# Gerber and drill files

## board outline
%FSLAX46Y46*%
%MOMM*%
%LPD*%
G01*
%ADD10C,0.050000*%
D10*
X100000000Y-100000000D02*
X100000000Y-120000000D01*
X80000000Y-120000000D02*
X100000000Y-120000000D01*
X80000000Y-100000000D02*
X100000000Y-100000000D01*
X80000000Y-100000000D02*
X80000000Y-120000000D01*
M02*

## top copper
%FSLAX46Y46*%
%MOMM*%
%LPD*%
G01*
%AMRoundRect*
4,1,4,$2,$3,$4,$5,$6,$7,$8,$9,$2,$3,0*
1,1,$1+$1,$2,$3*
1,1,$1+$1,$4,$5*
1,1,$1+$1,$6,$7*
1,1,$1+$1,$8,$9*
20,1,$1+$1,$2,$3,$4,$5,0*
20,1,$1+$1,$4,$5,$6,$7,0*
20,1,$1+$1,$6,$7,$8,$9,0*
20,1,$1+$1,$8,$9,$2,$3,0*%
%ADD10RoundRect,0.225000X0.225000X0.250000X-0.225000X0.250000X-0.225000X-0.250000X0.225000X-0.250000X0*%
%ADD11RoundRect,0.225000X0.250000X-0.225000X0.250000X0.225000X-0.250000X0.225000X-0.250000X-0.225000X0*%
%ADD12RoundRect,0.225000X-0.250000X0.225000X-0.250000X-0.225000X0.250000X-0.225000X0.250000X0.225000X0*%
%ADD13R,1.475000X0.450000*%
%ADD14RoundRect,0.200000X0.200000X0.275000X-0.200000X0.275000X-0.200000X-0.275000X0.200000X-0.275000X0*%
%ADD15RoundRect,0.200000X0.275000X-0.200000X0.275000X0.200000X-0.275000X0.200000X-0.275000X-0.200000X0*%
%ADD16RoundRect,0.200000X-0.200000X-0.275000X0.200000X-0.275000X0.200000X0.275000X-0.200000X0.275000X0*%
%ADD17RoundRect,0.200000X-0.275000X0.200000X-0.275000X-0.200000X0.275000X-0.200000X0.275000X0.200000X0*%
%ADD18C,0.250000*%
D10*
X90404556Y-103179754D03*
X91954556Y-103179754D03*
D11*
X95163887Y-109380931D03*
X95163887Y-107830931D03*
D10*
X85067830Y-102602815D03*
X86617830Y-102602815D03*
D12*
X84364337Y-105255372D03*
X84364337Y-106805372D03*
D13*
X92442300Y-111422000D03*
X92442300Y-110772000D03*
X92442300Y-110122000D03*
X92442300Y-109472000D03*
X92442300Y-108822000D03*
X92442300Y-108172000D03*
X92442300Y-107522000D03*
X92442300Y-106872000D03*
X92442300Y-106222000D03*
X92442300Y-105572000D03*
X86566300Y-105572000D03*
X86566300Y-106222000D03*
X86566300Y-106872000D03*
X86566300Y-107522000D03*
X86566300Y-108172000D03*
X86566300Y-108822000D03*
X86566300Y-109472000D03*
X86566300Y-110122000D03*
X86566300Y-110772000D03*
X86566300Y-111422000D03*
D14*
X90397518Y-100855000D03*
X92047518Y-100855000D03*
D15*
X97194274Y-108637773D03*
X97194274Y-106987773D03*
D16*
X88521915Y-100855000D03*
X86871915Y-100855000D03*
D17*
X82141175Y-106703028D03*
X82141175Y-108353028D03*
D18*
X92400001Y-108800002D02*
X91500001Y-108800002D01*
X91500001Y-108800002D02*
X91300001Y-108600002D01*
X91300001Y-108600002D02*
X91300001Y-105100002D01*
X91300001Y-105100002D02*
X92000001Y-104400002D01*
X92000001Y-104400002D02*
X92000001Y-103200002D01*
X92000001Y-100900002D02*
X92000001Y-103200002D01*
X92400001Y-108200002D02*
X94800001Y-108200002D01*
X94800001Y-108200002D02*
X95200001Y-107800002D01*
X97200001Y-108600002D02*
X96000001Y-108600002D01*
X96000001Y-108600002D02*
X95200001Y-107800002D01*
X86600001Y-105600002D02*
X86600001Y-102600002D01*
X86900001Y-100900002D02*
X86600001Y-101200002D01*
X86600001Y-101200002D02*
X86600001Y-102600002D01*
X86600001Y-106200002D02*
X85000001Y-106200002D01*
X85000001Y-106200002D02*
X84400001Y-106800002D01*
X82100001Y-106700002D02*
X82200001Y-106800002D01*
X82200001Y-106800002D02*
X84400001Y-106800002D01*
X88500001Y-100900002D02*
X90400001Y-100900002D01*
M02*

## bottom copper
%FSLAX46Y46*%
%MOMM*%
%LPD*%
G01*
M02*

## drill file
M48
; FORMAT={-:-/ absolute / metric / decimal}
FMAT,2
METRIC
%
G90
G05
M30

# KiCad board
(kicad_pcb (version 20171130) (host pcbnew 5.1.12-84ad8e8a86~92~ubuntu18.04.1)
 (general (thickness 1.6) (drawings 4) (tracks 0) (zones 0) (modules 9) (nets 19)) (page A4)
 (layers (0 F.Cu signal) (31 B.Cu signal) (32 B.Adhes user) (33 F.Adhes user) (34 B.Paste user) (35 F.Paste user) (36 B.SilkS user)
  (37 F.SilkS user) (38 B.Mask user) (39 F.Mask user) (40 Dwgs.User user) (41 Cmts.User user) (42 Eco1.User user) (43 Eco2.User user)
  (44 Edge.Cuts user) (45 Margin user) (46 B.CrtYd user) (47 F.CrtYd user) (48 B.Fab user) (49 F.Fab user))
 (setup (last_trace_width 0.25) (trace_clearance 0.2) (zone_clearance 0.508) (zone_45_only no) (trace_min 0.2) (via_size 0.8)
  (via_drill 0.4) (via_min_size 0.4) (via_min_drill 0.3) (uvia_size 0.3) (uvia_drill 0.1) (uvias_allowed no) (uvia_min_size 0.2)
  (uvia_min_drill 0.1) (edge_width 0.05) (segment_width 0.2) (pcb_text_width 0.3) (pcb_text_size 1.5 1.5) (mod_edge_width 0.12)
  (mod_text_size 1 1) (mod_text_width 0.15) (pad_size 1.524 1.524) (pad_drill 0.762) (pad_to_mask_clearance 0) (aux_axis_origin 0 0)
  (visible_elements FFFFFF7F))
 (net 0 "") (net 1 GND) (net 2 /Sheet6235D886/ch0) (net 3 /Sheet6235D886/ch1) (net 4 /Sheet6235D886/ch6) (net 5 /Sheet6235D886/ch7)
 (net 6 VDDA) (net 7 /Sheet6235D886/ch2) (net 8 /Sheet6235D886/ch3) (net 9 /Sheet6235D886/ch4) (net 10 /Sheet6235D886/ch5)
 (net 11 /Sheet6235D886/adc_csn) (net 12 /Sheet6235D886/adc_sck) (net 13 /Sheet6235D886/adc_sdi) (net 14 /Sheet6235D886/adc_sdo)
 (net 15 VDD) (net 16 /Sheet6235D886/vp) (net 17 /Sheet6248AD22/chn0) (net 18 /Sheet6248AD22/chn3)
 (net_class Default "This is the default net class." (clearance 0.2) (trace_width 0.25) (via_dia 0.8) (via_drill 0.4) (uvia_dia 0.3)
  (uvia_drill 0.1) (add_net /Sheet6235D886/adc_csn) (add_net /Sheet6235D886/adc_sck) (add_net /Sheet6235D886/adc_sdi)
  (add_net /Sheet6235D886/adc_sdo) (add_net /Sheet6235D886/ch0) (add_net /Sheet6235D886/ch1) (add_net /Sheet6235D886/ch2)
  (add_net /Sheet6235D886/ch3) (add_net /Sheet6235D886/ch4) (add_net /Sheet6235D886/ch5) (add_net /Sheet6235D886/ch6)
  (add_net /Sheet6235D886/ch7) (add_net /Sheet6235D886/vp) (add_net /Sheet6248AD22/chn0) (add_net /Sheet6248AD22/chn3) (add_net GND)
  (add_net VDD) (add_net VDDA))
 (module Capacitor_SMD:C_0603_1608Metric (layer F.Cu) (at 91.179556 103.179754 180.000000)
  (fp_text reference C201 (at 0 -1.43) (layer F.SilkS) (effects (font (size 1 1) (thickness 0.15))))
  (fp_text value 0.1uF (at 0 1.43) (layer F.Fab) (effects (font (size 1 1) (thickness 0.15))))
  (pad 2 smd roundrect (at 0.775 0 180.000000) (size 0.9 0.95) (layers F.Cu F.Mask F.Paste) (roundrect_rratio 0.25) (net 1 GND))
  (pad 1 smd roundrect (at -0.775 0 180.000000) (size 0.9 0.95) (layers F.Cu F.Mask F.Paste) (roundrect_rratio 0.25)
   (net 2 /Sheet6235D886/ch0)))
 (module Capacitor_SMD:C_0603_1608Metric (layer F.Cu) (at 95.163887 108.605931 90.000000)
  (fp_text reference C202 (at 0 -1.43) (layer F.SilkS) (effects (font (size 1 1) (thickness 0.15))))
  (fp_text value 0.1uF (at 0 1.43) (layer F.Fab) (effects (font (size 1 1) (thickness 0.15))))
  (pad 1 smd roundrect (at -0.775 0 90.000000) (size 0.9 0.95) (layers F.Cu F.Mask F.Paste) (roundrect_rratio 0.25) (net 1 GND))
  (pad 2 smd roundrect (at 0.775 0 90.000000) (size 0.9 0.95) (layers F.Cu F.Mask F.Paste) (roundrect_rratio 0.25)
   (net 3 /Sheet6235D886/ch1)))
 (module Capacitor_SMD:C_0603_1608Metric (layer F.Cu) (at 85.842830 102.602815 180.000000)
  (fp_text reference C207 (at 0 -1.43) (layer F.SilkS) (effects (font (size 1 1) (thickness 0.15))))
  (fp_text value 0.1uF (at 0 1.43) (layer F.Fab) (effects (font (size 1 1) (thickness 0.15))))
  (pad 2 smd roundrect (at 0.775 0 180.000000) (size 0.9 0.95) (layers F.Cu F.Mask F.Paste) (roundrect_rratio 0.25) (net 1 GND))
  (pad 1 smd roundrect (at -0.775 0 180.000000) (size 0.9 0.95) (layers F.Cu F.Mask F.Paste) (roundrect_rratio 0.25)
   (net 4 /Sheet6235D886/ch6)))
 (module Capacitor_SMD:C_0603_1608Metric (layer F.Cu) (at 84.364337 106.030372 270.000000)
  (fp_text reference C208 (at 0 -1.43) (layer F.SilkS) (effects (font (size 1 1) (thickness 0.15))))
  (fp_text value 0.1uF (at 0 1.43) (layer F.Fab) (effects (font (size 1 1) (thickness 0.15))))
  (pad 1 smd roundrect (at -0.775 0 270.000000) (size 0.9 0.95) (layers F.Cu F.Mask F.Paste) (roundrect_rratio 0.25) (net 1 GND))
  (pad 2 smd roundrect (at 0.775 0 270.000000) (size 0.9 0.95) (layers F.Cu F.Mask F.Paste) (roundrect_rratio 0.25)
   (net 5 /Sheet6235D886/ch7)))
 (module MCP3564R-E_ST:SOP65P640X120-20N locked (layer F.Cu) (at 89.504300 108.497000 180.000000)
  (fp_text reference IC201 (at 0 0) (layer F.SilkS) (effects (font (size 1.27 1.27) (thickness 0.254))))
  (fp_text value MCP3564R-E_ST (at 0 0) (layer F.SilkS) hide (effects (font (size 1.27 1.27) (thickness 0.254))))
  (pad 1 smd rect (at -2.938 -2.925 270.000000) (size 0.45 1.475) (layers F.Cu F.Mask F.Paste) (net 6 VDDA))
  (pad 2 smd rect (at -2.938 -2.275 270.000000) (size 0.45 1.475) (layers F.Cu F.Mask F.Paste) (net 1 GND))
  (pad 3 smd rect (at -2.938 -1.625 270.000000) (size 0.45 1.475) (layers F.Cu F.Mask F.Paste) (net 1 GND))
  (pad 4 smd rect (at -2.938 -0.975 270.000000) (size 0.45 1.475) (layers F.Cu F.Mask F.Paste))
  (pad 5 smd rect (at -2.938 -0.325 270.000000) (size 0.45 1.475) (layers F.Cu F.Mask F.Paste) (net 2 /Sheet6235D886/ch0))
  (pad 6 smd rect (at -2.938 0.325 270.000000) (size 0.45 1.475) (layers F.Cu F.Mask F.Paste) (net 3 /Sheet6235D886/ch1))
  (pad 7 smd rect (at -2.938 0.975 270.000000) (size 0.45 1.475) (layers F.Cu F.Mask F.Paste) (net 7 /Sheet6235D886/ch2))
  (pad 8 smd rect (at -2.938 1.625 270.000000) (size 0.45 1.475) (layers F.Cu F.Mask F.Paste) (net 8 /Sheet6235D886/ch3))
  (pad 9 smd rect (at -2.938 2.275 270.000000) (size 0.45 1.475) (layers F.Cu F.Mask F.Paste) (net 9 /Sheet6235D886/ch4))
  (pad 10 smd rect (at -2.938 2.925 270.000000) (size 0.45 1.475) (layers F.Cu F.Mask F.Paste) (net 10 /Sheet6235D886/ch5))
  (pad 11 smd rect (at 2.938 2.925 270.000000) (size 0.45 1.475) (layers F.Cu F.Mask F.Paste) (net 4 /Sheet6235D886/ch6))
  (pad 12 smd rect (at 2.938 2.275 270.000000) (size 0.45 1.475) (layers F.Cu F.Mask F.Paste) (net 5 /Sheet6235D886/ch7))
  (pad 13 smd rect (at 2.938 1.625 270.000000) (size 0.45 1.475) (layers F.Cu F.Mask F.Paste) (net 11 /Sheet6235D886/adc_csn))
  (pad 14 smd rect (at 2.938 0.975 270.000000) (size 0.45 1.475) (layers F.Cu F.Mask F.Paste) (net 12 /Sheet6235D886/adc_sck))
  (pad 15 smd rect (at 2.938 0.325 270.000000) (size 0.45 1.475) (layers F.Cu F.Mask F.Paste) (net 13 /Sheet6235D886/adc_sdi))
  (pad 16 smd rect (at 2.938 -0.325 270.000000) (size 0.45 1.475) (layers F.Cu F.Mask F.Paste) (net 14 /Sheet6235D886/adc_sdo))
  (pad 17 smd rect (at 2.938 -0.975 270.000000) (size 0.45 1.475) (layers F.Cu F.Mask F.Paste))
  (pad 18 smd rect (at 2.938 -1.625 270.000000) (size 0.45 1.475) (layers F.Cu F.Mask F.Paste))
  (pad 19 smd rect (at 2.938 -2.275 270.000000) (size 0.45 1.475) (layers F.Cu F.Mask F.Paste) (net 1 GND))
  (pad 20 smd rect (at 2.938 -2.925 270.000000) (size 0.45 1.475) (layers F.Cu F.Mask F.Paste) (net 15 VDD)))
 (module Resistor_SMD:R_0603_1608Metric (layer F.Cu) (at 91.222518 100.855000 180.000000)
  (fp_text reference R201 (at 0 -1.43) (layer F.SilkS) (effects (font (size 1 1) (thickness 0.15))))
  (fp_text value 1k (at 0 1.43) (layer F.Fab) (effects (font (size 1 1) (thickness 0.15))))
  (pad 2 smd roundrect (at 0.825 0 180.000000) (size 0.8 0.95) (layers F.Cu F.Mask F.Paste) (roundrect_rratio 0.25)
   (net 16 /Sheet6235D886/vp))
  (pad 1 smd roundrect (at -0.825 0 180.000000) (size 0.8 0.95) (layers F.Cu F.Mask F.Paste) (roundrect_rratio 0.25)
   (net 2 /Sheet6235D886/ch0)))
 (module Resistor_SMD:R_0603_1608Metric (layer F.Cu) (at 97.194274 107.812773 90.000000)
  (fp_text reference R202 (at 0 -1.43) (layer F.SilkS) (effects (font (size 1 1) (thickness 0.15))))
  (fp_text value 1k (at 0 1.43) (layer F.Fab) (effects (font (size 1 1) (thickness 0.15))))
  (pad 1 smd roundrect (at -0.825 0 90.000000) (size 0.8 0.95) (layers F.Cu F.Mask F.Paste) (roundrect_rratio 0.25)
   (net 3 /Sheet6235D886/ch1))
  (pad 2 smd roundrect (at 0.825 0 90.000000) (size 0.8 0.95) (layers F.Cu F.Mask F.Paste) (roundrect_rratio 0.25)
   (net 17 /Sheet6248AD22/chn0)))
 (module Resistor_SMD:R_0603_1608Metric (layer F.Cu) (at 87.696915 100.855000)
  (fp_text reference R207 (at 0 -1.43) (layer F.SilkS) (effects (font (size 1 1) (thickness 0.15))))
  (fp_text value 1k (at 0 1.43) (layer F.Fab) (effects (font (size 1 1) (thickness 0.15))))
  (pad 2 smd roundrect (at 0.825 0) (size 0.8 0.95) (layers F.Cu F.Mask F.Paste) (roundrect_rratio 0.25) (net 16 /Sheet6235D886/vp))
  (pad 1 smd roundrect (at -0.825 0) (size 0.8 0.95) (layers F.Cu F.Mask F.Paste) (roundrect_rratio 0.25) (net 4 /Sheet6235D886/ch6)))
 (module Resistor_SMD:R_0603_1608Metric (layer F.Cu) (at 82.141175 107.528028 270.000000)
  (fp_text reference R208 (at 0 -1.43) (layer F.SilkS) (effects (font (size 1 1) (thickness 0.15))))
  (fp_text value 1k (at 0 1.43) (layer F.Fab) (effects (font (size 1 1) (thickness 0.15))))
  (pad 1 smd roundrect (at -0.825 0 270.000000) (size 0.8 0.95) (layers F.Cu F.Mask F.Paste) (roundrect_rratio 0.25)
   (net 5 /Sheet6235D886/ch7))
  (pad 2 smd roundrect (at 0.825 0 270.000000) (size 0.8 0.95) (layers F.Cu F.Mask F.Paste) (roundrect_rratio 0.25)
   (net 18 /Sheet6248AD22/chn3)))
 (gr_line (start 100 100) (end 100 120) (layer Edge.Cuts) (width 0.05))
 (gr_line (start 80 120) (end 100 120) (layer Edge.Cuts) (width 0.05))
 (gr_line (start 80 100) (end 100 100) (layer Edge.Cuts) (width 0.05))
 (gr_line (start 80 100) (end 80 120) (layer Edge.Cuts) (width 0.05))
 (segment (start 92.400001 108.800002) (end 91.500001 108.800002) (width 0.250000) (layer F.Cu) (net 2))
 (segment (start 91.500001 108.800002) (end 91.300001 108.600002) (width 0.250000) (layer F.Cu) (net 2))
 (segment (start 91.300001 108.600002) (end 91.300001 105.100002) (width 0.250000) (layer F.Cu) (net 2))
 (segment (start 91.300001 105.100002) (end 92.000001 104.400002) (width 0.250000) (layer F.Cu) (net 2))
 (segment (start 92.000001 104.400002) (end 92.000001 103.200002) (width 0.250000) (layer F.Cu) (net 2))
 (segment (start 92.000001 100.900002) (end 92.000001 103.200002) (width 0.250000) (layer F.Cu) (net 2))
 (segment (start 92.400001 108.200002) (end 94.800001 108.200002) (width 0.250000) (layer F.Cu) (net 3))
 (segment (start 94.800001 108.200002) (end 95.200001 107.800002) (width 0.250000) (layer F.Cu) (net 3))
 (segment (start 97.200001 108.600002) (end 96.000001 108.600002) (width 0.250000) (layer F.Cu) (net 3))
 (segment (start 96.000001 108.600002) (end 95.200001 107.800002) (width 0.250000) (layer F.Cu) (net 3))
 (segment (start 86.600001 105.600002) (end 86.600001 102.600002) (width 0.250000) (layer F.Cu) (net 4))
 (segment (start 86.900001 100.900002) (end 86.600001 101.200002) (width 0.250000) (layer F.Cu) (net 4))
 (segment (start 86.600001 101.200002) (end 86.600001 102.600002) (width 0.250000) (layer F.Cu) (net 4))
 (segment (start 86.600001 106.200002) (end 85.000001 106.200002) (width 0.250000) (layer F.Cu) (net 5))
 (segment (start 85.000001 106.200002) (end 84.400001 106.800002) (width 0.250000) (layer F.Cu) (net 5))
 (segment (start 82.100001 106.700002) (end 82.200001 106.800002) (width 0.250000) (layer F.Cu) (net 5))
 (segment (start 82.200001 106.800002) (end 84.400001 106.800002) (width 0.250000) (layer F.Cu) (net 5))
 (segment (start 88.500001 100.900002) (end 90.400001 100.900002) (width 0.250000) (layer F.Cu) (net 16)))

